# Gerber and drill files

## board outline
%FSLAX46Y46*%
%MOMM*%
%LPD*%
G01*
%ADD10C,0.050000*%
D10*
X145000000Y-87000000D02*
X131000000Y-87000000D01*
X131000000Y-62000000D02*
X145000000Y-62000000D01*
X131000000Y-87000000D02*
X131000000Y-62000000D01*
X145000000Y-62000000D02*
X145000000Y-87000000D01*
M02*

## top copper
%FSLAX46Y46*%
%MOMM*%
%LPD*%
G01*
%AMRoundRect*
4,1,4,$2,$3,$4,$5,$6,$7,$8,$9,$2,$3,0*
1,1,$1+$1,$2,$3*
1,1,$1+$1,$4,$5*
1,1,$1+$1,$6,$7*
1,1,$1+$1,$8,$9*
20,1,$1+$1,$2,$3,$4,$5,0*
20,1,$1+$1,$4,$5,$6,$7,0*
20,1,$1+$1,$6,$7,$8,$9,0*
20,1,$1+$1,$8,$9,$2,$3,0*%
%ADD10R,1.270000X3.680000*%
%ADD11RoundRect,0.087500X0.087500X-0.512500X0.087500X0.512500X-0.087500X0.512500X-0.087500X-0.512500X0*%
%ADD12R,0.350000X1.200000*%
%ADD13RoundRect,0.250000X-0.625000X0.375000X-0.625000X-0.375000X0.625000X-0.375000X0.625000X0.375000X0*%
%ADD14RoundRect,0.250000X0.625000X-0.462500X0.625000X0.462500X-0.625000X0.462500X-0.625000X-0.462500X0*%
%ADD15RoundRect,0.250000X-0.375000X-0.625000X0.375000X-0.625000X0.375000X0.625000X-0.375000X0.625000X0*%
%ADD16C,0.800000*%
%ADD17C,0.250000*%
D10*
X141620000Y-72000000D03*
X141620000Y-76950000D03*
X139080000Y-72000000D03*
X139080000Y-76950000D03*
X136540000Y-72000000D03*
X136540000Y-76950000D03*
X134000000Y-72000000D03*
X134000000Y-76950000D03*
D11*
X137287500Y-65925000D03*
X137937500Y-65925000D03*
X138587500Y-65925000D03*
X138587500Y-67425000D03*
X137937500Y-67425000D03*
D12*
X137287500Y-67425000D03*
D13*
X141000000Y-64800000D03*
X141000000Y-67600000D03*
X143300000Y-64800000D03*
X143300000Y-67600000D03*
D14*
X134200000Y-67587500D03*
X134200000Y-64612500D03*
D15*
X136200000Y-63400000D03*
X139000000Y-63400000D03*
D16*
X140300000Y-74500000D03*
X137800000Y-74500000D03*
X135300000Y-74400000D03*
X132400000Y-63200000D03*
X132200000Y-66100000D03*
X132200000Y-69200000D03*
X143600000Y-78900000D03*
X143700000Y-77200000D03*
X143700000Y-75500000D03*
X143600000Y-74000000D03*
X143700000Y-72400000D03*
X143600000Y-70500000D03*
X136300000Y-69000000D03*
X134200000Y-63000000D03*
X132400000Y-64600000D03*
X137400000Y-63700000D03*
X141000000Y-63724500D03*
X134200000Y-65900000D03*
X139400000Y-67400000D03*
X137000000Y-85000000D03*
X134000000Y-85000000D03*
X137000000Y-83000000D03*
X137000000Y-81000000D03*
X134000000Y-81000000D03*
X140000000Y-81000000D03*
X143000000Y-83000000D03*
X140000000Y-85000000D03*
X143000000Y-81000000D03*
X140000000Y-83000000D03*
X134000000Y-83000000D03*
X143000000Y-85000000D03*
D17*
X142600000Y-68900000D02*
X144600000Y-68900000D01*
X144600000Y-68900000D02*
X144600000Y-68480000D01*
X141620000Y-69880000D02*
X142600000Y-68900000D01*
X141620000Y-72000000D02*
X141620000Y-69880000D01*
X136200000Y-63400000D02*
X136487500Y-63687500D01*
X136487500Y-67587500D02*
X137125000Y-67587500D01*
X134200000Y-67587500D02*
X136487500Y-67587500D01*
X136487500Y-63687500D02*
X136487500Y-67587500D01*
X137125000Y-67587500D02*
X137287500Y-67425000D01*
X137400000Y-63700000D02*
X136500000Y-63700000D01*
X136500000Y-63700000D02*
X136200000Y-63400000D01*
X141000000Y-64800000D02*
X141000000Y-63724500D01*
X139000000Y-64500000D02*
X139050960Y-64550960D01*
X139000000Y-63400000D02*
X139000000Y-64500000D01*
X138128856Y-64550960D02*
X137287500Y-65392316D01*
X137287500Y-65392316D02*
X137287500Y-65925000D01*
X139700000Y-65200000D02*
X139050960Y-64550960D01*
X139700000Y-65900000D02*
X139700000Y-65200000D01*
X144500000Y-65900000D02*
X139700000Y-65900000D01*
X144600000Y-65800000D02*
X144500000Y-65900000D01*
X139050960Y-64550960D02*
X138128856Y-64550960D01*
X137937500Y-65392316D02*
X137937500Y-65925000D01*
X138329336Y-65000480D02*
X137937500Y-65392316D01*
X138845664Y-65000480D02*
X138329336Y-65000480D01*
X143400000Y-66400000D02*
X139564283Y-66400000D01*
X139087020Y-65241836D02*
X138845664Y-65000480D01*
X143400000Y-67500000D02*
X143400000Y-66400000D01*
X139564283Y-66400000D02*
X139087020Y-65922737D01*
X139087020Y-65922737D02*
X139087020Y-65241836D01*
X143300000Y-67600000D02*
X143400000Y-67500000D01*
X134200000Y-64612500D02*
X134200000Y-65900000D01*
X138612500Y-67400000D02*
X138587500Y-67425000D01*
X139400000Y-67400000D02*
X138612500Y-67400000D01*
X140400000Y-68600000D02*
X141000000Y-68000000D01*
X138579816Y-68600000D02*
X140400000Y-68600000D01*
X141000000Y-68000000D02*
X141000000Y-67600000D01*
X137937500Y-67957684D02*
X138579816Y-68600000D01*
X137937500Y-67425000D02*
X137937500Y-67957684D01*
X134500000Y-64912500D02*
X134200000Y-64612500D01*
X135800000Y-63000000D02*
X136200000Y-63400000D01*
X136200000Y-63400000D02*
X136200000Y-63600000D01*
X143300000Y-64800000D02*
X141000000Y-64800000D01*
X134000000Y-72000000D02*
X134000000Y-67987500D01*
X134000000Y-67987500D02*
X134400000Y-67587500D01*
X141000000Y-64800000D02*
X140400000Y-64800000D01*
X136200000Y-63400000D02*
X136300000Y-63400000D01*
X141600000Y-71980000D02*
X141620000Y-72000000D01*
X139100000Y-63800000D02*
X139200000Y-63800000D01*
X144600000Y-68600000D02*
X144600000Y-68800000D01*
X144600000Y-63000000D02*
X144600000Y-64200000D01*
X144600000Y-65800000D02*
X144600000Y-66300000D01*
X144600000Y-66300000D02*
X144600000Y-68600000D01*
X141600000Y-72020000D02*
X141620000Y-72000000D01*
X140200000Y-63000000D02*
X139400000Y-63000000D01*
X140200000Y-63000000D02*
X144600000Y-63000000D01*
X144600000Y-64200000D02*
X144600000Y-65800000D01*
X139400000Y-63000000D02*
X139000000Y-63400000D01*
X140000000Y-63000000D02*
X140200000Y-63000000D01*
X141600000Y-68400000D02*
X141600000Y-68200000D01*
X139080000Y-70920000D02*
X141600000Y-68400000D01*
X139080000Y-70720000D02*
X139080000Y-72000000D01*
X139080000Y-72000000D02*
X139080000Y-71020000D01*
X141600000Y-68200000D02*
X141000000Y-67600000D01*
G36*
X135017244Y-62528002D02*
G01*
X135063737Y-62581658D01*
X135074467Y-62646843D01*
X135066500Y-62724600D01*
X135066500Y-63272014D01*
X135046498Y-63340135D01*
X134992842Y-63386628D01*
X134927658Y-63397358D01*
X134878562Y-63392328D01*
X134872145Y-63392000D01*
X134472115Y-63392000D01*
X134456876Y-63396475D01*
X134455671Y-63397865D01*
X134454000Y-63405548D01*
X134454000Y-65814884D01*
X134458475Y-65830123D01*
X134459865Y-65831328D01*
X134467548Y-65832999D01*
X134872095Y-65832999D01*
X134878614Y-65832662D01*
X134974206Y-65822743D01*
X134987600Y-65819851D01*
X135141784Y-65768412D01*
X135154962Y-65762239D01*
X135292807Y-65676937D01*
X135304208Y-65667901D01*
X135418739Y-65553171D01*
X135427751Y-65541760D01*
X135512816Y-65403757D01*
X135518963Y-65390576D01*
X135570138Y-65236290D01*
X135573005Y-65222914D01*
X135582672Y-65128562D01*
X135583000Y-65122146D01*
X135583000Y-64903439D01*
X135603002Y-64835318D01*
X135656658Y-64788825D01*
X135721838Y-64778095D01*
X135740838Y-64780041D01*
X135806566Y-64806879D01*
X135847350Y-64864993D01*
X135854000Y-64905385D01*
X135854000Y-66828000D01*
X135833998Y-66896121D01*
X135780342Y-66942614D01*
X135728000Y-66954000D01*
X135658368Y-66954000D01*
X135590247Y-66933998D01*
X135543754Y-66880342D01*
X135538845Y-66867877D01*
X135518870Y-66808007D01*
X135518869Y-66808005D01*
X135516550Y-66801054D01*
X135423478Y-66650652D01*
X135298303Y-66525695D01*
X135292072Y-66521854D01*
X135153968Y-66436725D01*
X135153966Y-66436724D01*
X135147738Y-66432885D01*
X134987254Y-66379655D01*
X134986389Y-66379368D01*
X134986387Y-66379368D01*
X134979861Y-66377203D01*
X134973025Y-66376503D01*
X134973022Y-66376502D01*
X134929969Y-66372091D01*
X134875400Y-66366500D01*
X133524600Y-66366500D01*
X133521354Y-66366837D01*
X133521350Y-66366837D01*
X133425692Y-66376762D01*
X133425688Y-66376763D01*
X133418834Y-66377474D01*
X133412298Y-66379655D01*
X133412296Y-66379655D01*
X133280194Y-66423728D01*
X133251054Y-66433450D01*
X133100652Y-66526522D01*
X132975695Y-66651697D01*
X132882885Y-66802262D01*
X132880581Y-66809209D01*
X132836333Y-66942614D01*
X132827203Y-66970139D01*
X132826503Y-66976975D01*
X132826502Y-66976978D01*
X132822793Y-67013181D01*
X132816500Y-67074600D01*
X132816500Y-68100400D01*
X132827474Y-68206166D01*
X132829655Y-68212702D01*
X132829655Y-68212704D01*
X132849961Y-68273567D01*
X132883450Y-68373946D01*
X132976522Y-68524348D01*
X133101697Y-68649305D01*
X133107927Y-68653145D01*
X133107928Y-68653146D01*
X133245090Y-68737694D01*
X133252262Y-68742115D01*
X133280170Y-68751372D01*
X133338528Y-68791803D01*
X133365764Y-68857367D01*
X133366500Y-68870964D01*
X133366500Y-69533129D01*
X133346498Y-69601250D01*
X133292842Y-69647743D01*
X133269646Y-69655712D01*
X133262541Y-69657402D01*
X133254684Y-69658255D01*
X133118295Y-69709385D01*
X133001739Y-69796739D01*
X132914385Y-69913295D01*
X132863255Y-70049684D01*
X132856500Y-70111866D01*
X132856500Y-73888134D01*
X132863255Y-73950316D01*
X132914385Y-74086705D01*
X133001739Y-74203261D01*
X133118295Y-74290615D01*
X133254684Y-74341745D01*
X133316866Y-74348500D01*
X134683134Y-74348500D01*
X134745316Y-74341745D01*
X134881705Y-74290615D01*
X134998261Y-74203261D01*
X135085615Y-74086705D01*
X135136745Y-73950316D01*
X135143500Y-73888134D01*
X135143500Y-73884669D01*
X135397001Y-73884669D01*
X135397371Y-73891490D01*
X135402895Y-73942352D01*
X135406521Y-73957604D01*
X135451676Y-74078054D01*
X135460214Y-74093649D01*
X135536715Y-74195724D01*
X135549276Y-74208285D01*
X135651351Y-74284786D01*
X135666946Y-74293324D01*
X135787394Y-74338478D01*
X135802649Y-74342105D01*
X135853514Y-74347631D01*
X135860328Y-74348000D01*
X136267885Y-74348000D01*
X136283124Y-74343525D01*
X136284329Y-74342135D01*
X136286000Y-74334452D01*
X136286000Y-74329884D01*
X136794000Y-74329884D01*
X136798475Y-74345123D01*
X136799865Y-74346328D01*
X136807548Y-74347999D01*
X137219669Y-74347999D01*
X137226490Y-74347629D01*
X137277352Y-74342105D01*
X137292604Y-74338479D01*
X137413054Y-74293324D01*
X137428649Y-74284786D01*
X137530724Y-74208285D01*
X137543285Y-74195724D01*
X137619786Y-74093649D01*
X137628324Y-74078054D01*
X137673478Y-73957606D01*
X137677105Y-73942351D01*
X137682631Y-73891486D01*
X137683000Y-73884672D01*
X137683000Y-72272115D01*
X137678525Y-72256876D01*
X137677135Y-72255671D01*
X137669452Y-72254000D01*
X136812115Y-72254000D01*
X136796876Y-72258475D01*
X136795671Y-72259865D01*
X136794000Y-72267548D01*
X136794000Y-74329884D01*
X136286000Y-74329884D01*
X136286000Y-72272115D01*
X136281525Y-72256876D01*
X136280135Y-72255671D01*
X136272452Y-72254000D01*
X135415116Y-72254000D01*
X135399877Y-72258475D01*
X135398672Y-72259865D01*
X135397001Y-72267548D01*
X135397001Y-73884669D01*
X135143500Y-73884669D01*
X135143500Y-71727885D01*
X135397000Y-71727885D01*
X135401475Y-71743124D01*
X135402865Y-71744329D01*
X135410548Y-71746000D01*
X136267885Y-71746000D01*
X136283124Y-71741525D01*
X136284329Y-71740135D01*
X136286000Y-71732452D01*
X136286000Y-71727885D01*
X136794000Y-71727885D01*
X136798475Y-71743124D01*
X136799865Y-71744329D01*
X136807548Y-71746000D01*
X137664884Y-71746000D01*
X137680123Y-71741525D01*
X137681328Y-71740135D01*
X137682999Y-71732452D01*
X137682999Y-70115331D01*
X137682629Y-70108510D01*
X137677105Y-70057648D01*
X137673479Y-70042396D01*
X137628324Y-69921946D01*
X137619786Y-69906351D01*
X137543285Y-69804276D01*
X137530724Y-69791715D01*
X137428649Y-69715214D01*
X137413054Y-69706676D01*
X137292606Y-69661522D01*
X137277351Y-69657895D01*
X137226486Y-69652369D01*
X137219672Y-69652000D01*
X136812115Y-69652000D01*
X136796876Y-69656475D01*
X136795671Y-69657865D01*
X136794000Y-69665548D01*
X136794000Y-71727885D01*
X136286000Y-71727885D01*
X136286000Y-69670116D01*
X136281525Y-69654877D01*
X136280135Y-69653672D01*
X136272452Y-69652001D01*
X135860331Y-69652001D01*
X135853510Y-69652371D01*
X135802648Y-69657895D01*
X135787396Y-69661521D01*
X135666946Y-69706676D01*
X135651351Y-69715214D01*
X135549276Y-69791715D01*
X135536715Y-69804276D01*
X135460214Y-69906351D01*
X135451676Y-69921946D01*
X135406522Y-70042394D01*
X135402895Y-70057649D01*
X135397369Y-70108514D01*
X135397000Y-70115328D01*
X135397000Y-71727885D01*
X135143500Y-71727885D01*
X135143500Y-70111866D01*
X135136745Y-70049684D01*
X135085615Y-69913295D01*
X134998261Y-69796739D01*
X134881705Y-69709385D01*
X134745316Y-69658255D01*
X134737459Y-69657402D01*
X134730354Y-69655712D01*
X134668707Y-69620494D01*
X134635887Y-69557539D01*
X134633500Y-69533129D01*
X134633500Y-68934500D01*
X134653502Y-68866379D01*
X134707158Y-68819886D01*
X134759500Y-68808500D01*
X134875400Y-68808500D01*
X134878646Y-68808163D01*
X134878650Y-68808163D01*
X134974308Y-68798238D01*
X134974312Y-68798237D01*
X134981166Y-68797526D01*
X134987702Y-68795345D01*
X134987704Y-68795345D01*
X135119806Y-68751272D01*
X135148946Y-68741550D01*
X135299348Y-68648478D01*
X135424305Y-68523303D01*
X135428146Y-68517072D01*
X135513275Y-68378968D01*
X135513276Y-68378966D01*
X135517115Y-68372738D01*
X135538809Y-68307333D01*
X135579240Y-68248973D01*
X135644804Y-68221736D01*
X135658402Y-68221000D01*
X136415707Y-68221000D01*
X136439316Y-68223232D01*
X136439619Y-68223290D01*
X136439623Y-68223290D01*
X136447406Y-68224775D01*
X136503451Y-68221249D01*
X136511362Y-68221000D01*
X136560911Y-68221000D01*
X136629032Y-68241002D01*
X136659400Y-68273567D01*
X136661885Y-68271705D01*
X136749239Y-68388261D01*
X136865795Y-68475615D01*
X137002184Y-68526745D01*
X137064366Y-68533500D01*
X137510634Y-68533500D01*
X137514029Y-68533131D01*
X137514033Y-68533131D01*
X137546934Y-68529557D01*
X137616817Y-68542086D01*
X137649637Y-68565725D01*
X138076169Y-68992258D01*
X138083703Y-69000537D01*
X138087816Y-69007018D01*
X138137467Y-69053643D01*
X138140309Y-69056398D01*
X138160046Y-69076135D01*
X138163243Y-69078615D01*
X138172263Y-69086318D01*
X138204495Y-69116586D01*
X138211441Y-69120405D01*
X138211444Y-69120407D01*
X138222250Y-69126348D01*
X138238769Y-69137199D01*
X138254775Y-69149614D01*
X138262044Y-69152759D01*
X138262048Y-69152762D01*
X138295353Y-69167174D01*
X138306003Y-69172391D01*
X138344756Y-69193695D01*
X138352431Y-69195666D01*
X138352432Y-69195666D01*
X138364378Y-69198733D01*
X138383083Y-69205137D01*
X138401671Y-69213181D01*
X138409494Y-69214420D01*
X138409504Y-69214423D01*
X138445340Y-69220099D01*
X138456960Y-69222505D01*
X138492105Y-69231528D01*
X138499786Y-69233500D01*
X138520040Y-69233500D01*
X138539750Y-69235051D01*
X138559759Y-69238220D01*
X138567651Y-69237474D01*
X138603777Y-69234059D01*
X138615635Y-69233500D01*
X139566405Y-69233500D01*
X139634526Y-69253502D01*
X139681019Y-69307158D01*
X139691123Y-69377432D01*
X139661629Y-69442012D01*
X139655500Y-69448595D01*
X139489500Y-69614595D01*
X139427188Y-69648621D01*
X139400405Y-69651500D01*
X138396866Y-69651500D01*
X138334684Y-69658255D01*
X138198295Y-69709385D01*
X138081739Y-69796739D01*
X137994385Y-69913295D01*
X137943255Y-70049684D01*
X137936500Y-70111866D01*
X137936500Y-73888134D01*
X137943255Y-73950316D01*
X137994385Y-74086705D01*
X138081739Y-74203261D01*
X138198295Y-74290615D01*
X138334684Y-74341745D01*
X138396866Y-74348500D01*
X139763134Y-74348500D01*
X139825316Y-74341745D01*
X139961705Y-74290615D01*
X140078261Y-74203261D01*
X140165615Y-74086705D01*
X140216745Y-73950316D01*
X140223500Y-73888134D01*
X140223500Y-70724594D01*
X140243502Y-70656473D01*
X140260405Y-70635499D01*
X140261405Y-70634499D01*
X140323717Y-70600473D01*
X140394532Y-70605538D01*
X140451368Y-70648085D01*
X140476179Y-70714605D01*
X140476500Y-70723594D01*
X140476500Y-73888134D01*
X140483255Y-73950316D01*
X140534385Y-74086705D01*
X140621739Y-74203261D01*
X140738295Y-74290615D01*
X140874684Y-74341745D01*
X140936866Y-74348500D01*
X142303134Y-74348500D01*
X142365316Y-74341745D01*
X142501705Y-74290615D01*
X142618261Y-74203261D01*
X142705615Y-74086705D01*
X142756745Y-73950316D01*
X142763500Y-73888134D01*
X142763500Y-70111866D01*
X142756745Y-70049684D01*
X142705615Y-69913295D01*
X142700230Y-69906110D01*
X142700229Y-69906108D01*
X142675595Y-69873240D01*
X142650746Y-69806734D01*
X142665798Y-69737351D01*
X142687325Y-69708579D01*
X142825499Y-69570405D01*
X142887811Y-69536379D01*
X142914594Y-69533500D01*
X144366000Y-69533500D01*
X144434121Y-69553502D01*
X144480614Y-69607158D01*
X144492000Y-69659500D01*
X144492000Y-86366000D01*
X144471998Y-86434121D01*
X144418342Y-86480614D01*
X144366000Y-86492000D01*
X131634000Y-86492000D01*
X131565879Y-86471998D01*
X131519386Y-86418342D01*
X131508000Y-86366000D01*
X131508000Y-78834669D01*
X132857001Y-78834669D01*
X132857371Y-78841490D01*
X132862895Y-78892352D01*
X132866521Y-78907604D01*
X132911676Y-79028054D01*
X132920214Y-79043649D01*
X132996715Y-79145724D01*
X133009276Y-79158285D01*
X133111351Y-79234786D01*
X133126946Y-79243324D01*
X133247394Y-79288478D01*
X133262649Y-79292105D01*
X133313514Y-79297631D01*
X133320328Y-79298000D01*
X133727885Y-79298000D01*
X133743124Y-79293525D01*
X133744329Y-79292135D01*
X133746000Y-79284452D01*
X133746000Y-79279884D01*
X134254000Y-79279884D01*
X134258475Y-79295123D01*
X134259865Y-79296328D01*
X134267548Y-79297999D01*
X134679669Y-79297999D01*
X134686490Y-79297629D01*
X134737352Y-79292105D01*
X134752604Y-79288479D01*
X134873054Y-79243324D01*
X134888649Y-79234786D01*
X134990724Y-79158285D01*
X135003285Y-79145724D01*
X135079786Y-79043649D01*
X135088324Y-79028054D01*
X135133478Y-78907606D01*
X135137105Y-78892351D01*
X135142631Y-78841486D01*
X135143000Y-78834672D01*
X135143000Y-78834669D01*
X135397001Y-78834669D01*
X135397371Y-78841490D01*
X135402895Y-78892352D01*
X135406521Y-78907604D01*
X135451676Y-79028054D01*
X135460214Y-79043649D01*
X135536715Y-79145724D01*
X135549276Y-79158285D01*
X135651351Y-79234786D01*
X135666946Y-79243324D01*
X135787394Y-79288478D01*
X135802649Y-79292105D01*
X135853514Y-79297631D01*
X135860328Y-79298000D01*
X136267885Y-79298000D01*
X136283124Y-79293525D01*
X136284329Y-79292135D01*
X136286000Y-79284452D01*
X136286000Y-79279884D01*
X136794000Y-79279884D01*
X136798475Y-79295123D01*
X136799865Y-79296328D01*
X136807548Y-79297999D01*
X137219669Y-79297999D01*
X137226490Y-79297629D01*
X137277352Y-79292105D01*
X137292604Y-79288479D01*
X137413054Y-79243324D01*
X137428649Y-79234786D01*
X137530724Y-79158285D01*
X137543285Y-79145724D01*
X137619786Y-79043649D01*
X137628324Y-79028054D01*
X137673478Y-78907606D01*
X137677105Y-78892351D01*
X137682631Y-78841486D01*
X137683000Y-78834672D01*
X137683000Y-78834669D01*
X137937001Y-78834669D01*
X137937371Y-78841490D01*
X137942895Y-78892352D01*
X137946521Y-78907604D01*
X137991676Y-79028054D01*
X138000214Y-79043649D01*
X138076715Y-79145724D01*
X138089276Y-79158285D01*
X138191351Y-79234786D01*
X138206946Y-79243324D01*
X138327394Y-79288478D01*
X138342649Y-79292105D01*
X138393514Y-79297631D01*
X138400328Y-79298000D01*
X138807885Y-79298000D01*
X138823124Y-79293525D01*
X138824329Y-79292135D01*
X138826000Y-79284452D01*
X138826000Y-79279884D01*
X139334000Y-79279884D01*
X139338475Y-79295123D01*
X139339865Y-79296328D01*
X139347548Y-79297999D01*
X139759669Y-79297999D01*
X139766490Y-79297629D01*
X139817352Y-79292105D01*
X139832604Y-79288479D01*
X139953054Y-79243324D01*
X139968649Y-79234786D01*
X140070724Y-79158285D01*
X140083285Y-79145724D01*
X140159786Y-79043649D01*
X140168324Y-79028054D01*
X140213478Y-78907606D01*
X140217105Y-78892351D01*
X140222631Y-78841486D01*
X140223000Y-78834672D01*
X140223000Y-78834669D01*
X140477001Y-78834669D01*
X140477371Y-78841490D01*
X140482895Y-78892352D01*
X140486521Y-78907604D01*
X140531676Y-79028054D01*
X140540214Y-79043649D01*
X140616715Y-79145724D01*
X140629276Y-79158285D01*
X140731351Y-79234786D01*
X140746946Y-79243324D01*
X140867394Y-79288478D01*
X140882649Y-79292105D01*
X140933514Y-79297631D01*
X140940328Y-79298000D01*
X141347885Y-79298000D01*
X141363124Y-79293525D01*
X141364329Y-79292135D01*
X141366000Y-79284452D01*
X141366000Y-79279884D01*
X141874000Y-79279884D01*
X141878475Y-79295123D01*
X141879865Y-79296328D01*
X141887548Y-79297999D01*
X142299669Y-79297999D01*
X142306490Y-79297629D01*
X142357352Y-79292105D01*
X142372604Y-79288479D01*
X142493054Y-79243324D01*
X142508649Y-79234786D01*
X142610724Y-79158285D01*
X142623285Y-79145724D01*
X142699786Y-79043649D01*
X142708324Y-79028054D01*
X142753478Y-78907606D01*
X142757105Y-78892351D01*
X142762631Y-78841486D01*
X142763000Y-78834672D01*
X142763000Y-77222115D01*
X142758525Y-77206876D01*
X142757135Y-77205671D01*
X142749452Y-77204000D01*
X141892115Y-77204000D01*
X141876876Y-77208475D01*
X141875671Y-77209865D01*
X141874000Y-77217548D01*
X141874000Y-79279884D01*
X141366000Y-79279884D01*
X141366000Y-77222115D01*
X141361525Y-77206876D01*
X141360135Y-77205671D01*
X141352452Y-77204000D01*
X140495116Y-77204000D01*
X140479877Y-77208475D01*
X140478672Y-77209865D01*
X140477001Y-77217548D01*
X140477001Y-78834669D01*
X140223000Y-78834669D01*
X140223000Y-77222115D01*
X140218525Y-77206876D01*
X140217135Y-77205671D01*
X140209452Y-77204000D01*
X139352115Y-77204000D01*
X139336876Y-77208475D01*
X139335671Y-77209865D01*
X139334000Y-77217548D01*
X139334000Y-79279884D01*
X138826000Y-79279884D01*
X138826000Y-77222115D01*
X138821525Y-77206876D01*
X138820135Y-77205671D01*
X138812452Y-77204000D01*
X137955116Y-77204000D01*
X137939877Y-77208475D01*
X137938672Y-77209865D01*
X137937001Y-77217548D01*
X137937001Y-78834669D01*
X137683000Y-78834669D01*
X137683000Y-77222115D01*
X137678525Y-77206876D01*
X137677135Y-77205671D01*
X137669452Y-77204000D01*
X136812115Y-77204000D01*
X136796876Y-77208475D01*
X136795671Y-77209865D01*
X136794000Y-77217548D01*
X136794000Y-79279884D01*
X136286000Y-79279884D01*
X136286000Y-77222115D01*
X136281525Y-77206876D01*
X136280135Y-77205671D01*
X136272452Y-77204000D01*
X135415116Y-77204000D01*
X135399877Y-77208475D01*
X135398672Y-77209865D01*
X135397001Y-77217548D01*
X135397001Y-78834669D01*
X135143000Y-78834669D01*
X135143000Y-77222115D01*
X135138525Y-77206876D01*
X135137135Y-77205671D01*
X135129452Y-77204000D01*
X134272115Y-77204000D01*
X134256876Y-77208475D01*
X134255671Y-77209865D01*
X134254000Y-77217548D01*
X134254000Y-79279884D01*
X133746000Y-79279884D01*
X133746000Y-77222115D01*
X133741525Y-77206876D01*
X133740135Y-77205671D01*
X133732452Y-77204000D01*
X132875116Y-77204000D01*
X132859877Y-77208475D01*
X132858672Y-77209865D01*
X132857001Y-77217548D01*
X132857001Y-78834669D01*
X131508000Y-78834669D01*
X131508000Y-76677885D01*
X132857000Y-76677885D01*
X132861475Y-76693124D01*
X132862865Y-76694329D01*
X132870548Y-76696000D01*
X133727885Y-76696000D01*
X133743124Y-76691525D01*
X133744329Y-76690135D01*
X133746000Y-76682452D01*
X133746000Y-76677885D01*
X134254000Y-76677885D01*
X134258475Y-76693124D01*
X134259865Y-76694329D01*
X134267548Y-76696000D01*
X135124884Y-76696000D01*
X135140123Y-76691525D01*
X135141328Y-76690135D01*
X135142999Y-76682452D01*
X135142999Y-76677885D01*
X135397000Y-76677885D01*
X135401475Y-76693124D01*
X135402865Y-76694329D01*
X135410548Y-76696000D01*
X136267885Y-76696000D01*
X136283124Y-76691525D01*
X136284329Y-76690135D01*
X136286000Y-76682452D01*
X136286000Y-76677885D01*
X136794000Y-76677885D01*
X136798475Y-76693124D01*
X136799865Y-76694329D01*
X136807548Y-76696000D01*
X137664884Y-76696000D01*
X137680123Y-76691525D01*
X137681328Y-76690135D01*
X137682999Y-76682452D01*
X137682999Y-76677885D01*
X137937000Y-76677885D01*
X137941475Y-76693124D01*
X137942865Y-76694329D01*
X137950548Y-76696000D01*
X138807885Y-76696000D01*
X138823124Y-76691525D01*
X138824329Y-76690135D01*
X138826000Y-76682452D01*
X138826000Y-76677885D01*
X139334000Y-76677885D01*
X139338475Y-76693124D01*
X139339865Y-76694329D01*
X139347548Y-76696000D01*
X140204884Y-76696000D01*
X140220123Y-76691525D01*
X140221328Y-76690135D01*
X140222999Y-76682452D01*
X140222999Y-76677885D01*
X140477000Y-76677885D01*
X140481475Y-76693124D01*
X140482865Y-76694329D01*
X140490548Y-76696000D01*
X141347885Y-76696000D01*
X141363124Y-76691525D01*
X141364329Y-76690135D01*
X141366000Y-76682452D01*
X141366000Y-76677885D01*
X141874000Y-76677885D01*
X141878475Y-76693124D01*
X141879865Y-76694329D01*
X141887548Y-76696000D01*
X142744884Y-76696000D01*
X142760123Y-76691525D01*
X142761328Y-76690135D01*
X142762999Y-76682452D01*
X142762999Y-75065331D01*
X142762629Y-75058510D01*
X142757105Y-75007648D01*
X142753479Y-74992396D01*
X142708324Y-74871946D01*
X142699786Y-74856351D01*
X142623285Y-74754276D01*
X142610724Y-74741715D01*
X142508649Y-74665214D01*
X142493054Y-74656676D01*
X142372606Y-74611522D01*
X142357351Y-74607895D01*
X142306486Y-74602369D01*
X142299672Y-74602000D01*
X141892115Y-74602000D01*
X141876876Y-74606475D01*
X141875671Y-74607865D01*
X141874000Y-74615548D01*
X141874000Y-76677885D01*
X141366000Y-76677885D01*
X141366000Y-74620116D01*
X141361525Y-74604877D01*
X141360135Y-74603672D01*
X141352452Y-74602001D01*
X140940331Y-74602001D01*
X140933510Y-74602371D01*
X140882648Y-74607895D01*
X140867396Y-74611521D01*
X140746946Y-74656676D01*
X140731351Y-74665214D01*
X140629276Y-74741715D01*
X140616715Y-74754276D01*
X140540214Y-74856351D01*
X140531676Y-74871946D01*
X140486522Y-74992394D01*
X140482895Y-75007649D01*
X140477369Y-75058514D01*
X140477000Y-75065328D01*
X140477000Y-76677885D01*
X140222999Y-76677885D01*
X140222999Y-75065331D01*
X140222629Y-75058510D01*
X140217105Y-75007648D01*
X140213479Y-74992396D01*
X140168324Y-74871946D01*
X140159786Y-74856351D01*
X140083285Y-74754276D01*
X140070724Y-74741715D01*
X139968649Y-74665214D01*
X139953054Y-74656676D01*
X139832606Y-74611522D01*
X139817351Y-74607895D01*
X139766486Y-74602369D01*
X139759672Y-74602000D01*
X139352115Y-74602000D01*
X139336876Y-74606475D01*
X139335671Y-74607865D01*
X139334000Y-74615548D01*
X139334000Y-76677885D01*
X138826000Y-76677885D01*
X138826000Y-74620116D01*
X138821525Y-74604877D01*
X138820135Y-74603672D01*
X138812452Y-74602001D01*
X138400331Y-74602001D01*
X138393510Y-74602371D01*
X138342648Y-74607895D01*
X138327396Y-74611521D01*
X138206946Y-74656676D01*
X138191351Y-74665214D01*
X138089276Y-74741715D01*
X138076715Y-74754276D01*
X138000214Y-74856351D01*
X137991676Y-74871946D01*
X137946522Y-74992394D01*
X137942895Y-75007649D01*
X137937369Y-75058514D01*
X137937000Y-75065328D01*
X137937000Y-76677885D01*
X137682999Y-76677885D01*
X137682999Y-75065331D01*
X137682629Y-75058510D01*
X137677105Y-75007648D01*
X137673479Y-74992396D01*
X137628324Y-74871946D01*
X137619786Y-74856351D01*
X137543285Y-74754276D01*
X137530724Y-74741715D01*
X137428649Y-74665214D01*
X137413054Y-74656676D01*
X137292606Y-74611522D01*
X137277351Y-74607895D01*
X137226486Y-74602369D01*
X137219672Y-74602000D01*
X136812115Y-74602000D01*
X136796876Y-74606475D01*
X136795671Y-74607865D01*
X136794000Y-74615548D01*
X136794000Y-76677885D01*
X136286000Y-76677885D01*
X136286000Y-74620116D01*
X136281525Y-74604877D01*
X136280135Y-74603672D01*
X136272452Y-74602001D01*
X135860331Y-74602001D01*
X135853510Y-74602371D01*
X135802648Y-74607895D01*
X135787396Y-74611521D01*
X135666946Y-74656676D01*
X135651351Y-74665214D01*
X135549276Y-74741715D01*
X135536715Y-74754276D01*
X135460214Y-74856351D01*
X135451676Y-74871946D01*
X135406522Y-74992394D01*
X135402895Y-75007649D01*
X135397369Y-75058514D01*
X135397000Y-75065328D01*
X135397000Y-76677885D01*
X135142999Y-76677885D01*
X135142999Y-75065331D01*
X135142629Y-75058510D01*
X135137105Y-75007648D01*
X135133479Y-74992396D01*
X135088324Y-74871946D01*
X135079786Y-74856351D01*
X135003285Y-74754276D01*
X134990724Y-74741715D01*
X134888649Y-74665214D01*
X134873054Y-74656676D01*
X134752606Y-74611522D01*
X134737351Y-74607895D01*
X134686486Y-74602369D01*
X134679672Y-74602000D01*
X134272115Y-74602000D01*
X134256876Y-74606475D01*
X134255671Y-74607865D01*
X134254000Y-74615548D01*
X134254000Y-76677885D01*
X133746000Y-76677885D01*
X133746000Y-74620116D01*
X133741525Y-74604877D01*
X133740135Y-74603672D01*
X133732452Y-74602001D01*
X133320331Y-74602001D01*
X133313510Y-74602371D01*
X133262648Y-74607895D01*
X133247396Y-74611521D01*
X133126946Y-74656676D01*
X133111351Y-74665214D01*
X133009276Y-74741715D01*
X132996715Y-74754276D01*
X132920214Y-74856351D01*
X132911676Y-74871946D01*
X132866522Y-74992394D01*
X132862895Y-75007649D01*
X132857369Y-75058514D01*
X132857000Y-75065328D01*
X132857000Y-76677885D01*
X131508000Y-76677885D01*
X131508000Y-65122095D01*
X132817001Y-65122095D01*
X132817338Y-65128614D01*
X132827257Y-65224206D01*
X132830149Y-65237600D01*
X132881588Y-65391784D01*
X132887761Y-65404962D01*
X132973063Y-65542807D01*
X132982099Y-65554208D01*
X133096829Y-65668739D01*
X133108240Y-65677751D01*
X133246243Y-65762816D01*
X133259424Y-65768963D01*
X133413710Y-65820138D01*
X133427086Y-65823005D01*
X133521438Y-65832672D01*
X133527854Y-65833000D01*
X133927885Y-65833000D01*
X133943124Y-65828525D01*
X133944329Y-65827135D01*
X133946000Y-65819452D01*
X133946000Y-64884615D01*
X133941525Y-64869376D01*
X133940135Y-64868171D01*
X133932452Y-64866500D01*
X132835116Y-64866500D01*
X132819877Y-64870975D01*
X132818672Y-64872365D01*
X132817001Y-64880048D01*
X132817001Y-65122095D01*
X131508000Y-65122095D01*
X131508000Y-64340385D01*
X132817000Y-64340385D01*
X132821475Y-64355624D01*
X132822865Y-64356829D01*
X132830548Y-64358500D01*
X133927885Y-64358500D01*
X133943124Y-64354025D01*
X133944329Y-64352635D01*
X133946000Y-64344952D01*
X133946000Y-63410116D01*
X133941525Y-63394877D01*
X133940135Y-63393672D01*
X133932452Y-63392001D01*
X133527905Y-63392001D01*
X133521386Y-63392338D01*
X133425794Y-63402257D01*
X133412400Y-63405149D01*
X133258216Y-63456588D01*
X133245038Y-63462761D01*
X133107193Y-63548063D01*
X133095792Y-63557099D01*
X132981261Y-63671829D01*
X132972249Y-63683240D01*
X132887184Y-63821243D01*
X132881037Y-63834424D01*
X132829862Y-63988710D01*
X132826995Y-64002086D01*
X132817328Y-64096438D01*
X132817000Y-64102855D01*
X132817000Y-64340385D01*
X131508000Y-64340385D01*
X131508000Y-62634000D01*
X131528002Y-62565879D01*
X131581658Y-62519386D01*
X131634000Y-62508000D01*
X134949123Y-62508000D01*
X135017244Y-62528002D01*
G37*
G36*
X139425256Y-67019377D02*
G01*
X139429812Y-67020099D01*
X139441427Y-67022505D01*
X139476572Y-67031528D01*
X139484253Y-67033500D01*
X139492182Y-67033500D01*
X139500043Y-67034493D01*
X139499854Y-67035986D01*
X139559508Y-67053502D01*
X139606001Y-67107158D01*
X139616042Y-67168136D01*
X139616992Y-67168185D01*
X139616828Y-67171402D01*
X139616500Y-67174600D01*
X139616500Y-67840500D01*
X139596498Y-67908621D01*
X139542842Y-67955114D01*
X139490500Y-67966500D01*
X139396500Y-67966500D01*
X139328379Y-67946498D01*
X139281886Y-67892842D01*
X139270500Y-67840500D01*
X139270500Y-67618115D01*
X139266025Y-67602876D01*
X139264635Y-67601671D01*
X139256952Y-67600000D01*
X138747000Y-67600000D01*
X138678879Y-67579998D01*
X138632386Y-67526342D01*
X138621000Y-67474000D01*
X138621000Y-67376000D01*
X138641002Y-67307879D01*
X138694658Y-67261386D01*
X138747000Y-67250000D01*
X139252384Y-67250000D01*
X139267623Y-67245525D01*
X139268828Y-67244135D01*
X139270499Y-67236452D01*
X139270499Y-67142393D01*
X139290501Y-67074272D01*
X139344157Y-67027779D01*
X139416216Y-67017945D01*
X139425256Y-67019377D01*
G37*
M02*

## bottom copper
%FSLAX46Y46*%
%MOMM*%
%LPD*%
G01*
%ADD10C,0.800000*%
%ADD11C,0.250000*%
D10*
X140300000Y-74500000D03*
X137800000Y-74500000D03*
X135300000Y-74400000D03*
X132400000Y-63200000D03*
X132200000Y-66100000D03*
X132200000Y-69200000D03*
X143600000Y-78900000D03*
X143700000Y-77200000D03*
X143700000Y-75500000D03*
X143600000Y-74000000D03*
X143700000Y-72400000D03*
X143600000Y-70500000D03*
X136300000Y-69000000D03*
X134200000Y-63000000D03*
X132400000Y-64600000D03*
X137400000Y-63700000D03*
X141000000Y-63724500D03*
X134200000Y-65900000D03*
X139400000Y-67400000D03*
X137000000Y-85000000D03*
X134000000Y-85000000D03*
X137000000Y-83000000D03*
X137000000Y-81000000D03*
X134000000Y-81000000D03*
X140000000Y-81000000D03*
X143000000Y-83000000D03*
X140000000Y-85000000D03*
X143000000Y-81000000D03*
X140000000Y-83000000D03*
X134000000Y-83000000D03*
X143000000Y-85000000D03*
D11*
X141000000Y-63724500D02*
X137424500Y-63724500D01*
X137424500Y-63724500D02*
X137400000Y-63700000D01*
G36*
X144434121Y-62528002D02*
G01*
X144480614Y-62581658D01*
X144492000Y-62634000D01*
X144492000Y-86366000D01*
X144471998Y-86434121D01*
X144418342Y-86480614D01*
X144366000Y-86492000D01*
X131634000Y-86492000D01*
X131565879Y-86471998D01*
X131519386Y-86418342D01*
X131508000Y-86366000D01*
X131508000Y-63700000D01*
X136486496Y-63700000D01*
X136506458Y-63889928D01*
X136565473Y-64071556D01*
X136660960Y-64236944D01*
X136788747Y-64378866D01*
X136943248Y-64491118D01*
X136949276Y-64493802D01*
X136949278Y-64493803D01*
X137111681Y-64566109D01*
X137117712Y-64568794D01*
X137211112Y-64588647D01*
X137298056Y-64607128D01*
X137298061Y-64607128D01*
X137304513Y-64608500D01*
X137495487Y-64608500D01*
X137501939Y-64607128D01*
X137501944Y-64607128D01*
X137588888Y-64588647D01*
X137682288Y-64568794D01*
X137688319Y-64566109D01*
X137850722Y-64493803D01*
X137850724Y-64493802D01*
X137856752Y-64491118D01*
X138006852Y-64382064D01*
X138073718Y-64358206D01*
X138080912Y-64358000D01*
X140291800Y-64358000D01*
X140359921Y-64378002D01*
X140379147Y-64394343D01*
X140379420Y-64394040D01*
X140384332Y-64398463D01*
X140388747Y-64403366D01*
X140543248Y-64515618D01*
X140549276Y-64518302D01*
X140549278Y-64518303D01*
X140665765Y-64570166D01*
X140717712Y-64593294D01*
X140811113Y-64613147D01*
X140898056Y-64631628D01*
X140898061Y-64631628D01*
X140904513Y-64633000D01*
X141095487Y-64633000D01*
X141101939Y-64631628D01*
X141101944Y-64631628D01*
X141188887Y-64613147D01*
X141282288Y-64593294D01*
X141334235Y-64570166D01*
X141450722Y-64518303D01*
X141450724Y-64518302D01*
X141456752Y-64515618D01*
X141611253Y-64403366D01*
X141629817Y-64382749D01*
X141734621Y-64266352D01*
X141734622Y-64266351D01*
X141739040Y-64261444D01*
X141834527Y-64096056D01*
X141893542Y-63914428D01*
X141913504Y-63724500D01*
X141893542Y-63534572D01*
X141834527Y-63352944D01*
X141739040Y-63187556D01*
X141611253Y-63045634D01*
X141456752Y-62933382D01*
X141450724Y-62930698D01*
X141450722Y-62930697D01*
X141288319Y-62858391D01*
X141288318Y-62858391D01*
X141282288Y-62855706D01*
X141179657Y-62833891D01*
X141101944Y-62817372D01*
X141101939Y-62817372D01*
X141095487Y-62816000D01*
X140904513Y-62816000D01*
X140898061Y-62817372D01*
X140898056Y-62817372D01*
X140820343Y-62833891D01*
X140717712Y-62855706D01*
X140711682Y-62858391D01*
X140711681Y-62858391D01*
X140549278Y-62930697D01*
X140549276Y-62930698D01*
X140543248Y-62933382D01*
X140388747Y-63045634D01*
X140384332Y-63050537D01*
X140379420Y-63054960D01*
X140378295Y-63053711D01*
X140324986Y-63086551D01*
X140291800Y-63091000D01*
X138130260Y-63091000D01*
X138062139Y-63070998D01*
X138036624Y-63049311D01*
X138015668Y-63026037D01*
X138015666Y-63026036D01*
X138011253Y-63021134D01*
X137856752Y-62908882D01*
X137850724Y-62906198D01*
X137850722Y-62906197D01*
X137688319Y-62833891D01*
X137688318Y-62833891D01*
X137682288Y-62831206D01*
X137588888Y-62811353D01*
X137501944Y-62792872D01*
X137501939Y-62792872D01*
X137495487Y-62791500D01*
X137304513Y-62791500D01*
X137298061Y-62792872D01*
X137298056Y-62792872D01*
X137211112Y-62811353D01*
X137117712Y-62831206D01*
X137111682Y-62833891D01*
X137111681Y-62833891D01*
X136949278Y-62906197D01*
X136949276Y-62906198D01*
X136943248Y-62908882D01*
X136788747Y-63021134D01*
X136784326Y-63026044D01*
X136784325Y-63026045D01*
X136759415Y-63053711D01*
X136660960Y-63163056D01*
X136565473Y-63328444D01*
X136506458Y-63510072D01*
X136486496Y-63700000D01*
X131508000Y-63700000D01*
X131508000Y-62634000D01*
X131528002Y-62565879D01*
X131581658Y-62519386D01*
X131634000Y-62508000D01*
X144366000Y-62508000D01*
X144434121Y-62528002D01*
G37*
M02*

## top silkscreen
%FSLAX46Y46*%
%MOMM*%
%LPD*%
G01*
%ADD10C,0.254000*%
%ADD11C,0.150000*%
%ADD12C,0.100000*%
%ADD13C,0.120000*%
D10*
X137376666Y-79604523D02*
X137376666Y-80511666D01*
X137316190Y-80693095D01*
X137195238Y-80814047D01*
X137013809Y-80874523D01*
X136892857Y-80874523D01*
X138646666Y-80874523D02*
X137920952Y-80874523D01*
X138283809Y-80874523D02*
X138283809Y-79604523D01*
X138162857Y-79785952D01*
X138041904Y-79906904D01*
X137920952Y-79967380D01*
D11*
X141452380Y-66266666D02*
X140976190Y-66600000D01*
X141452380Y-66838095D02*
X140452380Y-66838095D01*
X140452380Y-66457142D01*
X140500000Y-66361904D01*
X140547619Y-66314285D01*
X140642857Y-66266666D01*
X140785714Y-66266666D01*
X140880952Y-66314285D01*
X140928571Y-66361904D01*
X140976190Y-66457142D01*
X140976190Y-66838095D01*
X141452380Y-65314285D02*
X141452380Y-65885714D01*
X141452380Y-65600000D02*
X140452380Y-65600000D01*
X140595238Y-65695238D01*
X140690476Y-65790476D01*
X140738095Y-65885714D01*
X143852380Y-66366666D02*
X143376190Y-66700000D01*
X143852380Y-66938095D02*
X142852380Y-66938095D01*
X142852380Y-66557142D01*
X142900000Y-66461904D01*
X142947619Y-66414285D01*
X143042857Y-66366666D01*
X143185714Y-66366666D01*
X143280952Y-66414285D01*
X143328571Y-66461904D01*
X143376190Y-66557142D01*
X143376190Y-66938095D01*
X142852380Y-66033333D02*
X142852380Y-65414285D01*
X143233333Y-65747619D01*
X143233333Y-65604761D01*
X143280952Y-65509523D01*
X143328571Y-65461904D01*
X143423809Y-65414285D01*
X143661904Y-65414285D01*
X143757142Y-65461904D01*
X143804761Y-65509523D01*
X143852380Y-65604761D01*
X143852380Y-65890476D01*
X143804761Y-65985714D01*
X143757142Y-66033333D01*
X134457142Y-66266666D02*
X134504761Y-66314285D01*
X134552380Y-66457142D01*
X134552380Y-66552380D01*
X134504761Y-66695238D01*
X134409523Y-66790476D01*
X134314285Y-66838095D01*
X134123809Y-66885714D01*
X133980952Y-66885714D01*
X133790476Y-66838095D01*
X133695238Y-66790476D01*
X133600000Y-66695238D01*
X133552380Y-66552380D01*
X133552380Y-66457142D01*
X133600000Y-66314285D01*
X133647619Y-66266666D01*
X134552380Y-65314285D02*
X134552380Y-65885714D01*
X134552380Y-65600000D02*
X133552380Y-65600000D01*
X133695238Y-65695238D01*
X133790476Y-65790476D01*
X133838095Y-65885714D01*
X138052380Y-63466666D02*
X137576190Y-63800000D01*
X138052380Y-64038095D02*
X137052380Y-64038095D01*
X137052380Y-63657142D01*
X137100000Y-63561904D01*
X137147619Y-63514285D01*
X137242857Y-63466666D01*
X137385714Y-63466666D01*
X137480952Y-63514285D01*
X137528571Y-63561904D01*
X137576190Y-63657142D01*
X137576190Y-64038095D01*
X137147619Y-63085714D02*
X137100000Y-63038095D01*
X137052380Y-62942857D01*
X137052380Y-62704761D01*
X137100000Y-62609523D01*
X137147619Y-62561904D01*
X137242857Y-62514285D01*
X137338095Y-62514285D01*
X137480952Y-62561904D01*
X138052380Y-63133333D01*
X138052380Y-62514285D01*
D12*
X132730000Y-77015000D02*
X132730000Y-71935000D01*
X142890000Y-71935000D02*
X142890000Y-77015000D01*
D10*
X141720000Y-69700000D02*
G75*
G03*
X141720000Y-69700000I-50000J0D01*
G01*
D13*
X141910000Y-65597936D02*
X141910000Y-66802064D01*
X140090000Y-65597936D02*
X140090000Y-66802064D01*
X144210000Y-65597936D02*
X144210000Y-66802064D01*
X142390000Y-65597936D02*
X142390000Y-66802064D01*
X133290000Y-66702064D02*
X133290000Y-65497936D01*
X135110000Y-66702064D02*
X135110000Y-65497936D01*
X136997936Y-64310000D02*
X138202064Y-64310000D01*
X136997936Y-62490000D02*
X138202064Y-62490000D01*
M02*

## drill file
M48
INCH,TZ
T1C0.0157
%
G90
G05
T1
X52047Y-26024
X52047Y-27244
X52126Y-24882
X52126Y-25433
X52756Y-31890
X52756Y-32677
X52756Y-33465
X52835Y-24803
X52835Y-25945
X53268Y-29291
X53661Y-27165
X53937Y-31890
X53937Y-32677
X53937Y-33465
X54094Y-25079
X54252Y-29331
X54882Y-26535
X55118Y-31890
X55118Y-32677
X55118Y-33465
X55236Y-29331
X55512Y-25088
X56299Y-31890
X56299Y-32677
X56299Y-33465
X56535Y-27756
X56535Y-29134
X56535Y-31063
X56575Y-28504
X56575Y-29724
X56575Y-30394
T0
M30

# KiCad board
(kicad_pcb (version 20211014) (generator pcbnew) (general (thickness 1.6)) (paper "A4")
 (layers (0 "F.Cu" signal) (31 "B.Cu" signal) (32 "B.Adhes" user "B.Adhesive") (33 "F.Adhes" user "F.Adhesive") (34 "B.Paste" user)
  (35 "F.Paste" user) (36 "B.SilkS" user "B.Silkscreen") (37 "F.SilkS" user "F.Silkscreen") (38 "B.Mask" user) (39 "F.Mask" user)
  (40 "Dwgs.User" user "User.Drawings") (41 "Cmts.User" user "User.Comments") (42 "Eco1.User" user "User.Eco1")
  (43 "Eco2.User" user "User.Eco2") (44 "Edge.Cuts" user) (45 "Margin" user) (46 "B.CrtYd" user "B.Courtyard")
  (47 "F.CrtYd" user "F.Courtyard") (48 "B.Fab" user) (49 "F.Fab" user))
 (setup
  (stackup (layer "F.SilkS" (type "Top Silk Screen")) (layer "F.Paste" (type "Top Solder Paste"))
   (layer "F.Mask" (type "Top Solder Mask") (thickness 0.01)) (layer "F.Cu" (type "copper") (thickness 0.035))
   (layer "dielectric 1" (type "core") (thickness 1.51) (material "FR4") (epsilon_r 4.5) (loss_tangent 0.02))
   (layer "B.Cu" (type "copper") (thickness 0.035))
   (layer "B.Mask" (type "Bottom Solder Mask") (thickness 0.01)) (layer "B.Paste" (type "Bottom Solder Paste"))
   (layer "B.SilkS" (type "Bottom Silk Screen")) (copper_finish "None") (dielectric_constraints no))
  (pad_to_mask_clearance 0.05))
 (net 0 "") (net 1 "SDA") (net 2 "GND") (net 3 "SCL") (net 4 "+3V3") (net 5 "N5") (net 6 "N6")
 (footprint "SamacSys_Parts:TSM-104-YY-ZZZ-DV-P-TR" (layer "F.Cu") (at 137.81 74.475)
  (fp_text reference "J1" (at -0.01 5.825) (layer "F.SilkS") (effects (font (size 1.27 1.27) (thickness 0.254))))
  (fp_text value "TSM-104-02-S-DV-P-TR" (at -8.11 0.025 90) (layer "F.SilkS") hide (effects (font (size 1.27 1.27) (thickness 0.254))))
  (fp_line (start -5.08 2.54) (end -5.08 -2.54) (layer "F.SilkS") (width 0.1))
  (fp_line (start 5.08 -2.54) (end 5.08 2.54) (layer "F.SilkS") (width 0.1))
  (fp_circle (center 3.86 -4.775) (end 3.81 -4.775) (layer "F.SilkS") (width 0.254) (fill none))
  (pad "1" smd rect locked (at 3.81 -2.475) (size 1.27 3.68) (layers "F.Cu" "F.Paste" "F.Mask") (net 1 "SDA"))
  (pad "2" smd rect locked (at 3.81 2.475) (size 1.27 3.68) (layers "F.Cu" "F.Paste" "F.Mask") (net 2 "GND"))
  (pad "3" smd rect locked (at 1.27 -2.475) (size 1.27 3.68) (layers "F.Cu" "F.Paste" "F.Mask") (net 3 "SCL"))
  (pad "4" smd rect locked (at 1.27 2.475) (size 1.27 3.68) (layers "F.Cu" "F.Paste" "F.Mask") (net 2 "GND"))
  (pad "5" smd rect locked (at -1.27 -2.475) (size 1.27 3.68) (layers "F.Cu" "F.Paste" "F.Mask") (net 2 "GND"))
  (pad "6" smd rect locked (at -1.27 2.475) (size 1.27 3.68) (layers "F.Cu" "F.Paste" "F.Mask") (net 2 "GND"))
  (pad "7" smd rect locked (at -3.81 -2.475) (size 1.27 3.68) (layers "F.Cu" "F.Paste" "F.Mask") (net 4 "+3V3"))
  (pad "8" smd rect locked (at -3.81 2.475) (size 1.27 3.68) (layers "F.Cu" "F.Paste" "F.Mask") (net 2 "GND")))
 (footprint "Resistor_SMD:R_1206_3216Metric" (layer "F.Cu") (at 141 66.2 -90)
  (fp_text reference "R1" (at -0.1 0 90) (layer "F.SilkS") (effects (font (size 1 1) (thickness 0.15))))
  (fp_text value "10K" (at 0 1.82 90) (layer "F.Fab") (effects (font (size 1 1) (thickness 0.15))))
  (fp_line (start -0.602064 -0.91) (end 0.602064 -0.91) (layer "F.SilkS") (width 0.12))
  (fp_line (start -0.602064 0.91) (end 0.602064 0.91) (layer "F.SilkS") (width 0.12))
  (pad "1" smd roundrect locked (at -1.4 0 270) (size 1.25 1.75) (layers "F.Cu" "F.Paste" "F.Mask") (roundrect_rratio 0.2) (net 4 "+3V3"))
  (pad "2" smd roundrect locked (at 1.4 0 270) (size 1.25 1.75) (layers "F.Cu" "F.Paste" "F.Mask") (roundrect_rratio 0.2) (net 3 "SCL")))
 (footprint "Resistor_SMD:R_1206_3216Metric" (layer "F.Cu") (at 143.3 66.2 -90)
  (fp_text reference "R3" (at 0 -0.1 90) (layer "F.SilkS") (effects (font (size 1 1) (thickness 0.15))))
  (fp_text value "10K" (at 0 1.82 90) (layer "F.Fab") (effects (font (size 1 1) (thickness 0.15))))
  (fp_line (start -0.602064 -0.91) (end 0.602064 -0.91) (layer "F.SilkS") (width 0.12))
  (fp_line (start -0.602064 0.91) (end 0.602064 0.91) (layer "F.SilkS") (width 0.12))
  (pad "1" smd roundrect locked (at -1.4 0 270) (size 1.25 1.75) (layers "F.Cu" "F.Paste" "F.Mask") (roundrect_rratio 0.2) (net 4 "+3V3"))
  (pad "2" smd roundrect locked (at 1.4 0 270) (size 1.25 1.75) (layers "F.Cu" "F.Paste" "F.Mask") (roundrect_rratio 0.2) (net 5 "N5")))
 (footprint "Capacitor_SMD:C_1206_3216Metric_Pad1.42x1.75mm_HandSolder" (layer "F.Cu") (at 134.2 66.1 90)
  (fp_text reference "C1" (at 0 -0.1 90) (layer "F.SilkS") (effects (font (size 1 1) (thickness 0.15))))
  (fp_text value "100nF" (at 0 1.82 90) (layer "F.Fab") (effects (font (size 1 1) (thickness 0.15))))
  (fp_line (start -0.602064 -0.91) (end 0.602064 -0.91) (layer "F.SilkS") (width 0.12))
  (fp_line (start -0.602064 0.91) (end 0.602064 0.91) (layer "F.SilkS") (width 0.12))
  (pad "1" smd roundrect locked (at -1.4875 0 90) (size 1.425 1.75) (layers "F.Cu" "F.Paste" "F.Mask") (roundrect_rratio 0.1754385965)
   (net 4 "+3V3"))
  (pad "2" smd roundrect locked (at 1.4875 0 90) (size 1.425 1.75) (layers "F.Cu" "F.Paste" "F.Mask") (roundrect_rratio 0.1754385965)
   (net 2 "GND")))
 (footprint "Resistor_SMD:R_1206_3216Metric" (layer "F.Cu") (at 137.6 63.4)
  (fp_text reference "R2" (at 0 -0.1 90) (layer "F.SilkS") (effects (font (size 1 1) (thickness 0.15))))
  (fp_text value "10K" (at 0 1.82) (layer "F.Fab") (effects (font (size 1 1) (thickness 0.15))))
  (fp_line (start -0.602064 0.91) (end 0.602064 0.91) (layer "F.SilkS") (width 0.12))
  (fp_line (start -0.602064 -0.91) (end 0.602064 -0.91) (layer "F.SilkS") (width 0.12))
  (pad "1" smd roundrect locked (at -1.4 0) (size 1.25 1.75) (layers "F.Cu" "F.Paste" "F.Mask") (roundrect_rratio 0.2) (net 4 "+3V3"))
  (pad "2" smd roundrect locked (at 1.4 0) (size 1.25 1.75) (layers "F.Cu" "F.Paste" "F.Mask") (roundrect_rratio 0.2) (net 1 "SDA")))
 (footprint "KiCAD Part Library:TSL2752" (layer "F.Cu") (at 137.0875 68.025 90)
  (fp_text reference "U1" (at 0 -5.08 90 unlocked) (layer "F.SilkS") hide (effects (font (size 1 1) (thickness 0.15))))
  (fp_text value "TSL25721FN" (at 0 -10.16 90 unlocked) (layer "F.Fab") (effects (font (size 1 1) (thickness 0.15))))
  (pad "1" smd rect (at 0.6 0.2 90) (size 1.2 0.35) (layers "F.Cu" "F.Paste" "F.Mask") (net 4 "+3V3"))
  (pad "2" smd roundrect (at 0.6 0.85 90) (size 1.2 0.35) (layers "F.Cu" "F.Paste" "F.Mask") (roundrect_rratio 0.25) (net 3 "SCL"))
  (pad "3" smd roundrect (at 0.6 1.5 90) (size 1.2 0.35) (layers "F.Cu" "F.Paste" "F.Mask") (roundrect_rratio 0.25) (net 2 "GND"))
  (pad "4" smd roundrect (at 2.1 1.5 90) (size 1.2 0.35) (layers "F.Cu" "F.Paste" "F.Mask") (roundrect_rratio 0.25) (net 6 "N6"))
  (pad "5" smd roundrect (at 2.1 0.85 90) (size 1.2 0.35) (layers "F.Cu" "F.Paste" "F.Mask") (roundrect_rratio 0.25) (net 5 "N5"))
  (pad "6" smd roundrect (at 2.1 0.2 90) (size 1.2 0.35) (layers "F.Cu" "F.Paste" "F.Mask") (roundrect_rratio 0.25) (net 1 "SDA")))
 (gr_line (start 145 87) (end 131 87) (layer "Edge.Cuts") (width 0.05))
 (gr_line (start 131 62) (end 145 62) (layer "Edge.Cuts") (width 0.05))
 (gr_line (start 131 87) (end 131 62) (layer "Edge.Cuts") (width 0.05))
 (gr_line (start 145 62) (end 145 87) (layer "Edge.Cuts") (width 0.05))
 (segment (start 138.6125 67.4) (end 138.5875 67.425) (width 0.25) (layer "F.Cu") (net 2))
 (segment (start 134.2 64.6125) (end 134.2 65.9) (width 0.25) (layer "F.Cu") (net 2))
 (segment (start 134.5 64.9125) (end 134.2 64.6125) (width 0.25) (layer "F.Cu") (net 2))
 (segment (start 139.4 67.4) (end 138.6125 67.4) (width 0.25) (layer "F.Cu") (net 2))
 (via (at 132.2 69.2) (size 0.8) (drill 0.4) (layers "F.Cu" "B.Cu") (free) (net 2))
 (via (at 132.4 63.2) (size 0.8) (drill 0.4) (layers "F.Cu" "B.Cu") (free) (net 2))
 (via (at 137.8 74.5) (size 0.8) (drill 0.4) (layers "F.Cu" "B.Cu") (free) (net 2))
 (via (at 134.2 65.9) (size 0.8) (drill 0.4) (layers "F.Cu" "B.Cu") (free) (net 2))
 (via (at 135.3 74.4) (size 0.8) (drill 0.4) (layers "F.Cu" "B.Cu") (free) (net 2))
 (via (at 137 85) (size 0.8) (drill 0.4) (layers "F.Cu" "B.Cu") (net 2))
 (via (at 143.6 74) (size 0.8) (drill 0.4) (layers "F.Cu" "B.Cu") (free) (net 2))
 (via (at 134 85) (size 0.8) (drill 0.4) (layers "F.Cu" "B.Cu") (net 2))
 (via (at 140.3 74.5) (size 0.8) (drill 0.4) (layers "F.Cu" "B.Cu") (free) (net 2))
 (via (at 137 83) (size 0.8) (drill 0.4) (layers "F.Cu" "B.Cu") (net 2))
 (via (at 143.6 70.5) (size 0.8) (drill 0.4) (layers "F.Cu" "B.Cu") (free) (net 2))
 (via (at 137 81) (size 0.8) (drill 0.4) (layers "F.Cu" "B.Cu") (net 2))
 (via (at 134 81) (size 0.8) (drill 0.4) (layers "F.Cu" "B.Cu") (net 2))
 (via (at 143.6 78.9) (size 0.8) (drill 0.4) (layers "F.Cu" "B.Cu") (free) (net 2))
 (via (at 134.2 63) (size 0.8) (drill 0.4) (layers "F.Cu" "B.Cu") (free) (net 2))
 (via (at 132.4 64.6) (size 0.8) (drill 0.4) (layers "F.Cu" "B.Cu") (free) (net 2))
 (via (at 140 81) (size 0.8) (drill 0.4) (layers "F.Cu" "B.Cu") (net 2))
 (via (at 143.7 72.4) (size 0.8) (drill 0.4) (layers "F.Cu" "B.Cu") (free) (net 2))
 (via (at 143 83) (size 0.8) (drill 0.4) (layers "F.Cu" "B.Cu") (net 2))
 (via (at 140 85) (size 0.8) (drill 0.4) (layers "F.Cu" "B.Cu") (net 2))
 (via (at 143.7 77.2) (size 0.8) (drill 0.4) (layers "F.Cu" "B.Cu") (free) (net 2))
 (via (at 143 81) (size 0.8) (drill 0.4) (layers "F.Cu" "B.Cu") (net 2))
 (via (at 139.4 67.4) (size 0.8) (drill 0.4) (layers "F.Cu" "B.Cu") (free) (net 2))
 (via (at 140 83) (size 0.8) (drill 0.4) (layers "F.Cu" "B.Cu") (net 2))
 (via (at 134 83) (size 0.8) (drill 0.4) (layers "F.Cu" "B.Cu") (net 2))
 (via (at 143 85) (size 0.8) (drill 0.4) (layers "F.Cu" "B.Cu") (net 2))
 (via (at 132.2 66.1) (size 0.8) (drill 0.4) (layers "F.Cu" "B.Cu") (free) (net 2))
 (via (at 143.7 75.5) (size 0.8) (drill 0.4) (layers "F.Cu" "B.Cu") (free) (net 2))
 (via (at 136.3 69) (size 0.8) (drill 0.4) (layers "F.Cu" "B.Cu") (free) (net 2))
 (segment (start 135.8 63) (end 136.2 63.4) (width 0.25) (layer "F.Cu") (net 4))
 (segment (start 134.2 67.5875) (end 136.4875 67.5875) (width 0.25) (layer "F.Cu") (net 4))
 (segment (start 136.2 63.4) (end 136.2 63.6) (width 0.25) (layer "F.Cu") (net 4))
 (segment (start 143.3 64.8) (end 141 64.8) (width 0.25) (layer "F.Cu") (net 4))
 (segment (start 136.2 63.4) (end 136.4875 63.6875) (width 0.25) (layer "F.Cu") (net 4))
 (segment (start 134 72) (end 134 67.9875) (width 0.25) (layer "F.Cu") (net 4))
 (segment (start 134 67.9875) (end 134.4 67.5875) (width 0.25) (layer "F.Cu") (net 4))
 (segment (start 137.4 63.7) (end 136.5 63.7) (width 0.25) (layer "F.Cu") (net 4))
 (segment (start 136.4875 63.6875) (end 136.4875 67.5875) (width 0.25) (layer "F.Cu") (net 4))
 (segment (start 141 64.8) (end 141 63.7245) (width 0.25) (layer "F.Cu") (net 4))
 (segment (start 137.125 67.5875) (end 137.2875 67.425) (width 0.25) (layer "F.Cu") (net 4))
 (segment (start 136.4875 67.5875) (end 137.125 67.5875) (width 0.25) (layer "F.Cu") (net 4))
 (segment (start 141 64.8) (end 140.4 64.8) (width 0.25) (layer "F.Cu") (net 4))
 (segment (start 136.2 63.4) (end 136.3 63.4) (width 0.25) (layer "F.Cu") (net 4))
 (segment (start 136.5 63.7) (end 136.2 63.4) (width 0.25) (layer "F.Cu") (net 4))
 (via (at 141 63.7245) (size 0.8) (drill 0.4) (layers "F.Cu" "B.Cu") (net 4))
 (via (at 137.4 63.7) (size 0.8) (drill 0.4) (layers "F.Cu" "B.Cu") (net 4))
 (segment (start 141 63.7245) (end 137.4245 63.7245) (width 0.25) (layer "B.Cu") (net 4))
 (segment (start 137.4245 63.7245) (end 137.4 63.7) (width 0.25) (layer "B.Cu") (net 4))
 (segment (start 141.6 71.98) (end 141.62 72) (width 0.25) (layer "F.Cu") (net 1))
 (segment (start 139 64.5) (end 139.05096 64.55096) (width 0.25) (layer "F.Cu") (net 1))
 (segment (start 139.7 65.2) (end 139.05096 64.55096) (width 0.25) (layer "F.Cu") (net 1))
 (segment (start 141.62 69.88) (end 142.6 68.9) (width 0.25) (layer "F.Cu") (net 1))
 (segment (start 141.62 72) (end 141.62 69.88) (width 0.25) (layer "F.Cu") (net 1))
 (segment (start 139.1 63.8) (end 139.2 63.8) (width 0.25) (layer "F.Cu") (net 1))
 (segment (start 144.6 68.6) (end 144.6 68.8) (width 0.25) (layer "F.Cu") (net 1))
 (segment (start 144.6 63) (end 144.6 64.2) (width 0.25) (layer "F.Cu") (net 1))
 (segment (start 144.6 65.8) (end 144.6 66.3) (width 0.25) (layer "F.Cu") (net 1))
 (segment (start 139.7 65.9) (end 139.7 65.2) (width 0.25) (layer "F.Cu") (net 1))
 (segment (start 144.6 65.8) (end 144.5 65.9) (width 0.25) (layer "F.Cu") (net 1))
 (segment (start 144.6 66.3) (end 144.6 68.6) (width 0.25) (layer "F.Cu") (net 1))
 (segment (start 139 63.4) (end 139 64.5) (width 0.25) (layer "F.Cu") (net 1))
 (segment (start 141.6 72.02) (end 141.62 72) (width 0.25) (layer "F.Cu") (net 1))
 (segment (start 140.2 63) (end 139.4 63) (width 0.25) (layer "F.Cu") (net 1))
 (segment (start 144.6 68.9) (end 144.6 68.48) (width 0.25) (layer "F.Cu") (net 1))
 (segment (start 140.2 63) (end 144.6 63) (width 0.25) (layer "F.Cu") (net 1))
 (segment (start 144.6 64.2) (end 144.6 65.8) (width 0.25) (layer "F.Cu") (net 1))
 (segment (start 139.4 63) (end 139 63.4) (width 0.25) (layer "F.Cu") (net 1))
 (segment (start 142.6 68.9) (end 144.6 68.9) (width 0.25) (layer "F.Cu") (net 1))
 (segment (start 137.2875 65.392316) (end 137.2875 65.925) (width 0.25) (layer "F.Cu") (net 1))
 (segment (start 144.5 65.9) (end 139.7 65.9) (width 0.25) (layer "F.Cu") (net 1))
 (segment (start 140 63) (end 140.2 63) (width 0.25) (layer "F.Cu") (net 1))
 (segment (start 138.128856 64.55096) (end 137.2875 65.392316) (width 0.25) (layer "F.Cu") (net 1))
 (segment (start 139.05096 64.55096) (end 138.128856 64.55096) (width 0.25) (layer "F.Cu") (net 1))
 (segment (start 141.6 68.4) (end 141.6 68.2) (width 0.25) (layer "F.Cu") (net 3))
 (segment (start 139.08 70.92) (end 141.6 68.4) (width 0.25) (layer "F.Cu") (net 3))
 (segment (start 137.9375 67.957684) (end 138.579816 68.6) (width 0.25) (layer "F.Cu") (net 3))
 (segment (start 141 68) (end 141 67.6) (width 0.25) (layer "F.Cu") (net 3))
 (segment (start 137.9375 67.425) (end 137.9375 67.957684) (width 0.25) (layer "F.Cu") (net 3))
 (segment (start 138.579816 68.6) (end 140.4 68.6) (width 0.25) (layer "F.Cu") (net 3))
 (segment (start 139.08 70.72) (end 139.08 72) (width 0.25) (layer "F.Cu") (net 3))
 (segment (start 139.08 72) (end 139.08 71.02) (width 0.25) (layer "F.Cu") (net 3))
 (segment (start 140.4 68.6) (end 141 68) (width 0.25) (layer "F.Cu") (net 3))
 (segment (start 141.6 68.2) (end 141 67.6) (width 0.25) (layer "F.Cu") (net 3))
 (segment (start 137.9375 65.392316) (end 137.9375 65.925) (width 0.25) (layer "F.Cu") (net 5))
 (segment (start 143.3 67.6) (end 143.4 67.5) (width 0.25) (layer "F.Cu") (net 5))
 (segment (start 138.845664 65.00048) (end 138.329336 65.00048) (width 0.25) (layer "F.Cu") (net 5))
 (segment (start 139.564283 66.4) (end 139.08702 65.922737) (width 0.25) (layer "F.Cu") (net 5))
 (segment (start 138.329336 65.00048) (end 137.9375 65.392316) (width 0.25) (layer "F.Cu") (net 5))
 (segment (start 139.08702 65.241836) (end 138.845664 65.00048) (width 0.25) (layer "F.Cu") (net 5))
 (segment (start 143.4 66.4) (end 139.564283 66.4) (width 0.25) (layer "F.Cu") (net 5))
 (segment (start 143.4 67.5) (end 143.4 66.4) (width 0.25) (layer "F.Cu") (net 5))
 (segment (start 139.08702 65.922737) (end 139.08702 65.241836) (width 0.25) (layer "F.Cu") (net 5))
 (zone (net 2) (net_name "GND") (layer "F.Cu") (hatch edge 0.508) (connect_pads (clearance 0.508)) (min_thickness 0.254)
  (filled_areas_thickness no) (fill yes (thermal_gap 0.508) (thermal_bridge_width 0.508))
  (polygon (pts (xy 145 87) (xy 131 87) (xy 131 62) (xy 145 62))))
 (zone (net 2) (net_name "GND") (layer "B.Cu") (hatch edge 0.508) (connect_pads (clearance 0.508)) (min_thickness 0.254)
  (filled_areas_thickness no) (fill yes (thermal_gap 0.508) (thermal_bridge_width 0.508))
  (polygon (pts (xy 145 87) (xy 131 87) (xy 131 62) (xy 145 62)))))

